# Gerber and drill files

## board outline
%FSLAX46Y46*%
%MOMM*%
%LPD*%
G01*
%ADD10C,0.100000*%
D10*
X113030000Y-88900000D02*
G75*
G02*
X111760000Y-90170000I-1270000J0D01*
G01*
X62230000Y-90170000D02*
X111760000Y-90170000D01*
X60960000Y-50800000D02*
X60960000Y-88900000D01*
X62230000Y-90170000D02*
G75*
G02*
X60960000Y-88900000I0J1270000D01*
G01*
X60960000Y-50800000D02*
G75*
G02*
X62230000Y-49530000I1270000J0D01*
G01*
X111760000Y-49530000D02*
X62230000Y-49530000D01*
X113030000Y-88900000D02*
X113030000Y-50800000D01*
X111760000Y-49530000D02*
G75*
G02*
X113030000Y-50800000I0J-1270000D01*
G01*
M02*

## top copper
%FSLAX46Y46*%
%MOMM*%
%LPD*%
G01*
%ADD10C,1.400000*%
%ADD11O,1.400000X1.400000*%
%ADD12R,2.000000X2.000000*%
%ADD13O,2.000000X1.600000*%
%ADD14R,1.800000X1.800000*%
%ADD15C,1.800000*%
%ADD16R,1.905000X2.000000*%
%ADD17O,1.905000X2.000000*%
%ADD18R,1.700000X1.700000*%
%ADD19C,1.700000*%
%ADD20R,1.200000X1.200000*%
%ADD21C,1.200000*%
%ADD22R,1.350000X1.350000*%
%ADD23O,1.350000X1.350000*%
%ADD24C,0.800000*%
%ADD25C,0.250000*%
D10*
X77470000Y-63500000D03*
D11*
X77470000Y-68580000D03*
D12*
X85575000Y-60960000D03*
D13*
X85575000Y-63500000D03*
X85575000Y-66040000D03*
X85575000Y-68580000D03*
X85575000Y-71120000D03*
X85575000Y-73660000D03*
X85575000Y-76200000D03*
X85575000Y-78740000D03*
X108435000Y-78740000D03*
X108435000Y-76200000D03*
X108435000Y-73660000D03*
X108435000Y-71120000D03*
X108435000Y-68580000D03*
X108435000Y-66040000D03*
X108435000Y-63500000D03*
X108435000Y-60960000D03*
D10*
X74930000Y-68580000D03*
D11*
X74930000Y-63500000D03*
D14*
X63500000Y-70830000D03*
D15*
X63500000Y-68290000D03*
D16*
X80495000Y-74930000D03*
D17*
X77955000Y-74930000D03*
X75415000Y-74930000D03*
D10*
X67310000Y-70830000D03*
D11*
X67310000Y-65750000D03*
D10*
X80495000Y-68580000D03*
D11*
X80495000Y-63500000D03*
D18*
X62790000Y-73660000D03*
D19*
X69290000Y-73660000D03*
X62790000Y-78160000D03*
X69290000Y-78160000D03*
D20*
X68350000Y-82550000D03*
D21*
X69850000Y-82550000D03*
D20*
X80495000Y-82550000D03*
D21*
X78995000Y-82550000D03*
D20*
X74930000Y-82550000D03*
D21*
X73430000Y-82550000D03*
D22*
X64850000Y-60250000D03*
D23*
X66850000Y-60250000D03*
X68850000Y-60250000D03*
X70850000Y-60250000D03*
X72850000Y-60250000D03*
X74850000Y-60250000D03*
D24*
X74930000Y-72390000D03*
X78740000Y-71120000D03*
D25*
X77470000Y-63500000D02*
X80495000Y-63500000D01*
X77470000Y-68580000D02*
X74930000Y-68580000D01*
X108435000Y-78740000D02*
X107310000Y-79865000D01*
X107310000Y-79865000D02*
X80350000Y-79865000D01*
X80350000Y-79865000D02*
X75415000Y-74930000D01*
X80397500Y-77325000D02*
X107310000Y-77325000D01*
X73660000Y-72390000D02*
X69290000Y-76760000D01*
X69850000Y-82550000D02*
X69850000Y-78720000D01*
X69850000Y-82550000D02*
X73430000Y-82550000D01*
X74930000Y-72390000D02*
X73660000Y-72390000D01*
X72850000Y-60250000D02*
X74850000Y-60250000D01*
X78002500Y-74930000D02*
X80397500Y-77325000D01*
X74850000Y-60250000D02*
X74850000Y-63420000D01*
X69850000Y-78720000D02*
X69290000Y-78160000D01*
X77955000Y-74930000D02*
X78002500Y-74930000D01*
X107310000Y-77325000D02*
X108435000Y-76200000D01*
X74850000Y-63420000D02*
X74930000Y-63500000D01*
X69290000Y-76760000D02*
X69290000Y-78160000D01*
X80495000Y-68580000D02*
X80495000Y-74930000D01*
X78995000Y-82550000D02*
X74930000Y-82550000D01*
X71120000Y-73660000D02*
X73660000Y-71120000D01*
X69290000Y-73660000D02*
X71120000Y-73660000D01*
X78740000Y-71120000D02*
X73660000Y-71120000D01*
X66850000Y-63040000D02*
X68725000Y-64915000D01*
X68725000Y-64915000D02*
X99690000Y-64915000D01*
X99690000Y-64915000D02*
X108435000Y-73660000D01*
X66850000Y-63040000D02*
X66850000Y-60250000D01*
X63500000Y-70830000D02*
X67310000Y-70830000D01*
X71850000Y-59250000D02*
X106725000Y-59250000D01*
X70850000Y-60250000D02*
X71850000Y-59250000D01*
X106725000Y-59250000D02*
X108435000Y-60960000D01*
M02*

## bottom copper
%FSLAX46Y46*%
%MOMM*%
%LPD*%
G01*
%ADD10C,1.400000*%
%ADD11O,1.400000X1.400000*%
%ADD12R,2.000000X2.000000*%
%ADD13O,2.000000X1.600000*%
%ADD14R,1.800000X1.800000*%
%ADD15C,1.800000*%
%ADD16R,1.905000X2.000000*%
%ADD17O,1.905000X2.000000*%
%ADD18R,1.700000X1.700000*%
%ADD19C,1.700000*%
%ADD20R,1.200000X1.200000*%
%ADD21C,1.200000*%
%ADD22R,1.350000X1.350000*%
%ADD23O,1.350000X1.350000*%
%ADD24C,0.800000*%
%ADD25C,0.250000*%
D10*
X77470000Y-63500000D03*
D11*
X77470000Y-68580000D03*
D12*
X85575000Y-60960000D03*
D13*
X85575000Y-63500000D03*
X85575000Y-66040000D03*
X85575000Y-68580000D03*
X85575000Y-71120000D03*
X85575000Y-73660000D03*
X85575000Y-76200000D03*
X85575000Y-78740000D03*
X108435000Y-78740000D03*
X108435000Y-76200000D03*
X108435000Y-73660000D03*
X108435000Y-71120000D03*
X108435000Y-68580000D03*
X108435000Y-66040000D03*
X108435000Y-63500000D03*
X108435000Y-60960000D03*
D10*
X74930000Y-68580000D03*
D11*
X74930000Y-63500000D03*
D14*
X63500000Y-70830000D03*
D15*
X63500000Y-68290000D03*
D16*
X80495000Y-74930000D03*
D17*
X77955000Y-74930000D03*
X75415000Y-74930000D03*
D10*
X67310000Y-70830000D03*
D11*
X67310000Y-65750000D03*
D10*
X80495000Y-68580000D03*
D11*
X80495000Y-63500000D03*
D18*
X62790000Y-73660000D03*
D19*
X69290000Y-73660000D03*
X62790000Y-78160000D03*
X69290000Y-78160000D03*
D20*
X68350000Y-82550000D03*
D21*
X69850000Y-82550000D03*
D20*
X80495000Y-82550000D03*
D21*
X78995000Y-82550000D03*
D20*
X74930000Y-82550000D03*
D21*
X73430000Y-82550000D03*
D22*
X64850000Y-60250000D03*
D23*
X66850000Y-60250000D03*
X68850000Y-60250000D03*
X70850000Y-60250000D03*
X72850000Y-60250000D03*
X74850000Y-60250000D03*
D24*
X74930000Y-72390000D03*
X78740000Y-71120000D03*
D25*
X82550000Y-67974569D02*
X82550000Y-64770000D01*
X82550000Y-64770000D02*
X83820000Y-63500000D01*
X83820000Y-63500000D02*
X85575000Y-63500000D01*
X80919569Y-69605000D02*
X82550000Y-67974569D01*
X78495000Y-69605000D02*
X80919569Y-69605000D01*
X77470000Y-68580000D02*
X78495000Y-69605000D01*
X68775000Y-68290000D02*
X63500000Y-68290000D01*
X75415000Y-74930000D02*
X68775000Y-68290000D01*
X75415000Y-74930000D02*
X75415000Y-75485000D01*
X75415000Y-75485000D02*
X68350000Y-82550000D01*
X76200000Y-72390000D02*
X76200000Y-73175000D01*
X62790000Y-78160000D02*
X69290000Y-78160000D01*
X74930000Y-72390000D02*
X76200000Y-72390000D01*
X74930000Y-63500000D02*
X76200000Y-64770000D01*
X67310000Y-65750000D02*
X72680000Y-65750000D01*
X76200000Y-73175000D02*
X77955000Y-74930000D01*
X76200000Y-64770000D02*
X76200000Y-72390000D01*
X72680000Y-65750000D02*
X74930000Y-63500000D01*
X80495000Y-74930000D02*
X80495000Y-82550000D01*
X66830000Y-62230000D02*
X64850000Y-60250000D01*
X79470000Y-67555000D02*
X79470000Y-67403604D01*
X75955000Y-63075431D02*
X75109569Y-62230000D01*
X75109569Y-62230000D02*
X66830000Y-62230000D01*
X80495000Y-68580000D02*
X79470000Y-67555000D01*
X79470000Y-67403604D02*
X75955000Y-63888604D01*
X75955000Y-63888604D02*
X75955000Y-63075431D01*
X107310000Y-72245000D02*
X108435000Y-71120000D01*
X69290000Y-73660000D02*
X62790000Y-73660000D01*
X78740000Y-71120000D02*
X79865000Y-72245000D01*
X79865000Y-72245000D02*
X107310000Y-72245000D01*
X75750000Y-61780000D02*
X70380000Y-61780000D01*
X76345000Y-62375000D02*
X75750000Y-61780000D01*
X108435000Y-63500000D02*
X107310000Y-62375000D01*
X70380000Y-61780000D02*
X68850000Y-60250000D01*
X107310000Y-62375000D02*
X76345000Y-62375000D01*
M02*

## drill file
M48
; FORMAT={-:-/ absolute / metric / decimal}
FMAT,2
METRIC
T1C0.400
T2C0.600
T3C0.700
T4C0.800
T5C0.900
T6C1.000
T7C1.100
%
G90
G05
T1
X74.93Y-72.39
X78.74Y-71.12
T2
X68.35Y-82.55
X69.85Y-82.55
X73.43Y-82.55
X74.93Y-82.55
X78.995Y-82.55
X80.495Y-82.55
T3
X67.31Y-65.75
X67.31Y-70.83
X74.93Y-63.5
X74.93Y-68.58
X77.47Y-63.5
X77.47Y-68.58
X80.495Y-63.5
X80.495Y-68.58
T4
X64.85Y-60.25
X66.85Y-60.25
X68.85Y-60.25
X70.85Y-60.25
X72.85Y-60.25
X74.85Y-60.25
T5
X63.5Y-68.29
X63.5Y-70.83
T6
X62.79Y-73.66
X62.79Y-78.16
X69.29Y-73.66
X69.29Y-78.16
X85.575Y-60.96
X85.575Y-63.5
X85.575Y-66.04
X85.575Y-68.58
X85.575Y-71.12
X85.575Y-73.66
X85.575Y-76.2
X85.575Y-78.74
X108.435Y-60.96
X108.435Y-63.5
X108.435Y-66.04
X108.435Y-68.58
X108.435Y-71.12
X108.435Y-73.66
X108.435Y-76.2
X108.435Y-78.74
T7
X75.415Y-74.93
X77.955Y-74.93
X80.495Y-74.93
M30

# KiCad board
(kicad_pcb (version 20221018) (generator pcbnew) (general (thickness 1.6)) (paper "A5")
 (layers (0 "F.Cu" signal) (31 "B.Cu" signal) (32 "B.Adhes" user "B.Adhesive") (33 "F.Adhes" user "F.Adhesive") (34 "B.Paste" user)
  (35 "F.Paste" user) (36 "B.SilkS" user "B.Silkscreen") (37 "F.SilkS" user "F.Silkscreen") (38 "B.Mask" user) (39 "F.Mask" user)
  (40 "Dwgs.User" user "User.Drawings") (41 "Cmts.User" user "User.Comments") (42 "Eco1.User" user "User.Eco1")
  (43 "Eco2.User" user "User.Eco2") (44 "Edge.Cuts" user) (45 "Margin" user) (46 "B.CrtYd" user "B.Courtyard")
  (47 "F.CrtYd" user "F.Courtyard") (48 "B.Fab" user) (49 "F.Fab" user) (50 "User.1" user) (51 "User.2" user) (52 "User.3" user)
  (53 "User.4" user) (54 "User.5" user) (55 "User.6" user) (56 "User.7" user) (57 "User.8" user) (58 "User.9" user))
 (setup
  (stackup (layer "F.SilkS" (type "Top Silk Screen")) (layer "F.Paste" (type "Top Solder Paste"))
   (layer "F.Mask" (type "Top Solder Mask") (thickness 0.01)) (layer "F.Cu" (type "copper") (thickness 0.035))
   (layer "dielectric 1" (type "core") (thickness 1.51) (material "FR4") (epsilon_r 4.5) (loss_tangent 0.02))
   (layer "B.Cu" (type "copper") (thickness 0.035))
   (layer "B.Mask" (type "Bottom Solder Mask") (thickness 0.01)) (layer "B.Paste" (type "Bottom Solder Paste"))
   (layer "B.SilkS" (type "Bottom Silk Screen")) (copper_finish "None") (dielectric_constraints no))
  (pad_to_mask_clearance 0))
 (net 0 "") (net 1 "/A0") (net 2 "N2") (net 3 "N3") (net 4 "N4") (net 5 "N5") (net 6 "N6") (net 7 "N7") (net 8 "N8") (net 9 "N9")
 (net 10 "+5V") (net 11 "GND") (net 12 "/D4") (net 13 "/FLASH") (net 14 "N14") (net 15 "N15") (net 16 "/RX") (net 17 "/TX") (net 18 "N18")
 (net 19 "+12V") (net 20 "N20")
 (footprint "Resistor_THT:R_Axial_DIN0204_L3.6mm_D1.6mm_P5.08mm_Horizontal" (layer "F.Cu") (at 77.47 63.5 -90)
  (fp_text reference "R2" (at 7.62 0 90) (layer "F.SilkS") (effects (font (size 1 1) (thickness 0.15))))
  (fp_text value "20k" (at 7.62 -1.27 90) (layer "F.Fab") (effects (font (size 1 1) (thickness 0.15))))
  (pad "1" thru_hole circle (at 0 0 270) (size 1.4 1.4) (drill 0.7) (layers "*.Cu" "*.Mask") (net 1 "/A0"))
  (pad "2" thru_hole oval (at 5.08 0 270) (size 1.4 1.4) (drill 0.7) (layers "*.Cu" "*.Mask") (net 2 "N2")))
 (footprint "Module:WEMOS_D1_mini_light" (layer "F.Cu") (at 85.575 60.96)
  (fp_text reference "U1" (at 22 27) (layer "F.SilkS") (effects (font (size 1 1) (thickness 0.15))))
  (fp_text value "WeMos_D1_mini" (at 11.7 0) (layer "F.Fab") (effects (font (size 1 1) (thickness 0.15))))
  (pad "1" thru_hole rect (at 0 0) (size 2 2) (drill 1) (layers "*.Cu" "*.Mask") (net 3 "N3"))
  (pad "2" thru_hole oval (at 0 2.54) (size 2 1.6) (drill 1) (layers "*.Cu" "*.Mask") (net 1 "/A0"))
  (pad "3" thru_hole oval (at 0 5.08) (size 2 1.6) (drill 1) (layers "*.Cu" "*.Mask") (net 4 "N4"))
  (pad "4" thru_hole oval (at 0 7.62) (size 2 1.6) (drill 1) (layers "*.Cu" "*.Mask") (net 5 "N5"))
  (pad "5" thru_hole oval (at 0 10.16) (size 2 1.6) (drill 1) (layers "*.Cu" "*.Mask") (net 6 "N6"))
  (pad "6" thru_hole oval (at 0 12.7) (size 2 1.6) (drill 1) (layers "*.Cu" "*.Mask") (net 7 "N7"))
  (pad "7" thru_hole oval (at 0 15.24) (size 2 1.6) (drill 1) (layers "*.Cu" "*.Mask") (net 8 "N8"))
  (pad "8" thru_hole oval (at 0 17.78) (size 2 1.6) (drill 1) (layers "*.Cu" "*.Mask") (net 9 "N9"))
  (pad "9" thru_hole oval (at 22.86 17.78) (size 2 1.6) (drill 1) (layers "*.Cu" "*.Mask") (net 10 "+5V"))
  (pad "10" thru_hole oval (at 22.86 15.24) (size 2 1.6) (drill 1) (layers "*.Cu" "*.Mask") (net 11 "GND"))
  (pad "11" thru_hole oval (at 22.86 12.7) (size 2 1.6) (drill 1) (layers "*.Cu" "*.Mask") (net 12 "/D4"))
  (pad "12" thru_hole oval (at 22.86 10.16) (size 2 1.6) (drill 1) (layers "*.Cu" "*.Mask") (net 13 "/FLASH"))
  (pad "13" thru_hole oval (at 22.86 7.62) (size 2 1.6) (drill 1) (layers "*.Cu" "*.Mask") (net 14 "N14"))
  (pad "14" thru_hole oval (at 22.86 5.08) (size 2 1.6) (drill 1) (layers "*.Cu" "*.Mask") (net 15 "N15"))
  (pad "15" thru_hole oval (at 22.86 2.54) (size 2 1.6) (drill 1) (layers "*.Cu" "*.Mask") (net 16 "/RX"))
  (pad "16" thru_hole oval (at 22.86 0) (size 2 1.6) (drill 1) (layers "*.Cu" "*.Mask") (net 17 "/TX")))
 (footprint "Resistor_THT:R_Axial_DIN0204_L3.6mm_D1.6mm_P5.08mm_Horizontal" (layer "F.Cu") (at 74.93 68.58 90)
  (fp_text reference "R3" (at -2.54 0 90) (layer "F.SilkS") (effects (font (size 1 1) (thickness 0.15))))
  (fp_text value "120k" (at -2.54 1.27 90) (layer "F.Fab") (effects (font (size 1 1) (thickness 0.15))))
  (pad "1" thru_hole circle (at 0 0 90) (size 1.4 1.4) (drill 0.7) (layers "*.Cu" "*.Mask") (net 2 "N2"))
  (pad "2" thru_hole oval (at 5.08 0 90) (size 1.4 1.4) (drill 0.7) (layers "*.Cu" "*.Mask") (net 11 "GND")))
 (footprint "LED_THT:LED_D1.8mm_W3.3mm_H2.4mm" (layer "F.Cu") (at 63.5 70.83 90)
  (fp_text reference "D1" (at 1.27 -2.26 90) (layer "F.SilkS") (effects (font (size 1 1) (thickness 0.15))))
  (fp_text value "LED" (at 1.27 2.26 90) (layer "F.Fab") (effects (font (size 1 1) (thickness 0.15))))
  (pad "1" thru_hole rect (at 0 0 90) (size 1.8 1.8) (drill 0.9) (layers "*.Cu" "*.Mask") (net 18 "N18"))
  (pad "2" thru_hole circle (at 2.54 0 90) (size 1.8 1.8) (drill 0.9) (layers "*.Cu" "*.Mask") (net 10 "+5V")))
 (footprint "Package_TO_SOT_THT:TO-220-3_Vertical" (layer "F.Cu") (at 80.495 74.93 180)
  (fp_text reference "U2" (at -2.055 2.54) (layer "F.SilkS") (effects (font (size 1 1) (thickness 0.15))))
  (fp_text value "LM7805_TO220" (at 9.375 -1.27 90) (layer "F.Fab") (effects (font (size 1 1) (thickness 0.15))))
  (pad "1" thru_hole rect (at 0 0 180) (size 1.905 2) (drill 1.1) (layers "*.Cu" "*.Mask") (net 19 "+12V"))
  (pad "2" thru_hole oval (at 2.54 0 180) (size 1.905 2) (drill 1.1) (layers "*.Cu" "*.Mask") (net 11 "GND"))
  (pad "3" thru_hole oval (at 5.08 0 180) (size 1.905 2) (drill 1.1) (layers "*.Cu" "*.Mask") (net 10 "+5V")))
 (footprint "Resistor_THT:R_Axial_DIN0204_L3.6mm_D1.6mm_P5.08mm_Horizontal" (layer "F.Cu") (at 67.31 70.83 90)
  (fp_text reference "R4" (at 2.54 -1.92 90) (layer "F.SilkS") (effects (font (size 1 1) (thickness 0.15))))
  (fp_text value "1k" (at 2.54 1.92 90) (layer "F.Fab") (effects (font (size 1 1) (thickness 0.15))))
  (pad "1" thru_hole circle (at 0 0 90) (size 1.4 1.4) (drill 0.7) (layers "*.Cu" "*.Mask") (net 18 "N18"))
  (pad "2" thru_hole oval (at 5.08 0 90) (size 1.4 1.4) (drill 0.7) (layers "*.Cu" "*.Mask") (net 11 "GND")))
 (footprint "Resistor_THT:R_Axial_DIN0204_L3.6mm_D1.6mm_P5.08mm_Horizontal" (layer "F.Cu") (at 80.495 68.58 90)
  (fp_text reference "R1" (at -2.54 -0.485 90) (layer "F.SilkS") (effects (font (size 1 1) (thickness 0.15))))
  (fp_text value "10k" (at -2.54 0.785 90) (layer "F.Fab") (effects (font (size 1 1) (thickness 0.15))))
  (pad "1" thru_hole circle (at 0 0 90) (size 1.4 1.4) (drill 0.7) (layers "*.Cu" "*.Mask") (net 19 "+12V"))
  (pad "2" thru_hole oval (at 5.08 0 90) (size 1.4 1.4) (drill 0.7) (layers "*.Cu" "*.Mask") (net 1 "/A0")))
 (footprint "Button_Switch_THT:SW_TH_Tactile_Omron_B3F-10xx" (layer "F.Cu") (at 62.79 73.66)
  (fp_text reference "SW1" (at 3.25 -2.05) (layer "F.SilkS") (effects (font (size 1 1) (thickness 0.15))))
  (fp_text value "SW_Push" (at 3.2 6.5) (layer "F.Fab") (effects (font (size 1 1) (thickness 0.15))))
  (pad "1" thru_hole rect (at 0 0) (size 1.7 1.7) (drill 1) (layers "*.Cu" "*.Mask") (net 13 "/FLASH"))
  (pad "1" thru_hole circle (at 6.5 0) (size 1.7 1.7) (drill 1) (layers "*.Cu" "*.Mask") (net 13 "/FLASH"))
  (pad "2" thru_hole circle (at 0 4.5) (size 1.7 1.7) (drill 1) (layers "*.Cu" "*.Mask") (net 11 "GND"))
  (pad "2" thru_hole circle (at 6.5 4.5) (size 1.7 1.7) (drill 1) (layers "*.Cu" "*.Mask") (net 11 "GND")))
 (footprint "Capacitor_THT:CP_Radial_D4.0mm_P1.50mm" (layer "F.Cu") (at 68.35 82.55)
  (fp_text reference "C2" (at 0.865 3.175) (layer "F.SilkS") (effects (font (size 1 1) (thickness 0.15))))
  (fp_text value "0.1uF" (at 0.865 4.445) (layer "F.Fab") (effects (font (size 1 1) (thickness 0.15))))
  (pad "1" thru_hole rect (at 0 0) (size 1.2 1.2) (drill 0.6) (layers "*.Cu" "*.Mask") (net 10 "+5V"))
  (pad "2" thru_hole circle (at 1.5 0) (size 1.2 1.2) (drill 0.6) (layers "*.Cu" "*.Mask") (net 11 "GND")))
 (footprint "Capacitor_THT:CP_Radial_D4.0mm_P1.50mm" (layer "F.Cu") (at 80.495 82.55 180)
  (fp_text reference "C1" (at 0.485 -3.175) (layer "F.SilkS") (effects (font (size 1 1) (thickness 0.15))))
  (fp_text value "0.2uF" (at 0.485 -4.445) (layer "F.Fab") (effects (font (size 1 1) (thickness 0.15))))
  (pad "1" thru_hole rect (at 0 0 180) (size 1.2 1.2) (drill 0.6) (layers "*.Cu" "*.Mask") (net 19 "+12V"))
  (pad "2" thru_hole circle (at 1.5 0 180) (size 1.2 1.2) (drill 0.6) (layers "*.Cu" "*.Mask") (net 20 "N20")))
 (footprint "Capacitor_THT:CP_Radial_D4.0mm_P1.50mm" (layer "F.Cu") (at 74.93 82.55 180)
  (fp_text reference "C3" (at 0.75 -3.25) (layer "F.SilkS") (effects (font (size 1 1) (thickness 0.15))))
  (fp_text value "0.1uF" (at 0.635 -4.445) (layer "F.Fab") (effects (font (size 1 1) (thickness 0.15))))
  (pad "1" thru_hole rect (at 0 0 180) (size 1.2 1.2) (drill 0.6) (layers "*.Cu" "*.Mask") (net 20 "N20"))
  (pad "2" thru_hole circle (at 1.5 0 180) (size 1.2 1.2) (drill 0.6) (layers "*.Cu" "*.Mask") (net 11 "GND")))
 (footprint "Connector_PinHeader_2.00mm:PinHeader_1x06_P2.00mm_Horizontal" (layer "F.Cu") (at 64.85 60.25 90)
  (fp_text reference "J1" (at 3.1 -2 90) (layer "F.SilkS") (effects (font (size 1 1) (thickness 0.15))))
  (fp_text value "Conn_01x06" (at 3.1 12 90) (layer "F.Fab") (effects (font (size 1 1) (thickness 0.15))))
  (pad "1" thru_hole rect (at 0 0 90) (size 1.35 1.35) (drill 0.8) (layers "*.Cu" "*.Mask") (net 19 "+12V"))
  (pad "2" thru_hole oval (at 0 2 90) (size 1.35 1.35) (drill 0.8) (layers "*.Cu" "*.Mask") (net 12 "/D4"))
  (pad "3" thru_hole oval (at 0 4 90) (size 1.35 1.35) (drill 0.8) (layers "*.Cu" "*.Mask") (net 16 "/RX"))
  (pad "4" thru_hole oval (at 0 6 90) (size 1.35 1.35) (drill 0.8) (layers "*.Cu" "*.Mask") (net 17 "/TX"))
  (pad "5" thru_hole oval (at 0 8 90) (size 1.35 1.35) (drill 0.8) (layers "*.Cu" "*.Mask") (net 11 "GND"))
  (pad "6" thru_hole oval (at 0 10 90) (size 1.35 1.35) (drill 0.8) (layers "*.Cu" "*.Mask") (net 11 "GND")))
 (gr_arc locked (start 113.03 88.9) (mid 112.658026 89.798026) (end 111.76 90.17) (stroke (width 0.1) (type default)) (layer "Edge.Cuts"))
 (gr_line locked (start 62.23 90.17) (end 111.76 90.17) (stroke (width 0.1) (type default)) (layer "Edge.Cuts"))
 (gr_line locked (start 60.96 50.8) (end 60.96 88.9) (stroke (width 0.1) (type default)) (layer "Edge.Cuts"))
 (gr_arc locked (start 62.23 90.17) (mid 61.331974 89.798026) (end 60.96 88.9) (stroke (width 0.1) (type default)) (layer "Edge.Cuts"))
 (gr_arc locked (start 60.96 50.8) (mid 61.331974 49.901974) (end 62.23 49.53) (stroke (width 0.1) (type default)) (layer "Edge.Cuts"))
 (gr_line locked (start 111.76 49.53) (end 62.23 49.53) (stroke (width 0.1) (type default)) (layer "Edge.Cuts"))
 (gr_line locked (start 113.03 88.9) (end 113.03 50.8) (stroke (width 0.1) (type default)) (layer "Edge.Cuts"))
 (gr_arc locked (start 111.76 49.53) (mid 112.658026 49.901974) (end 113.03 50.8) (stroke (width 0.1) (type default)) (layer "Edge.Cuts"))
 (segment (start 77.47 63.5) (end 80.495 63.5) (width 0.25) (layer "F.Cu") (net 1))
 (segment (start 77.47 68.58) (end 74.93 68.58) (width 0.25) (layer "F.Cu") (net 1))
 (segment (start 82.55 67.974569) (end 82.55 64.77) (width 0.25) (layer "B.Cu") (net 1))
 (segment (start 82.55 64.77) (end 83.82 63.5) (width 0.25) (layer "B.Cu") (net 1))
 (segment (start 83.82 63.5) (end 85.575 63.5) (width 0.25) (layer "B.Cu") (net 1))
 (segment (start 80.919569 69.605) (end 82.55 67.974569) (width 0.25) (layer "B.Cu") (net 1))
 (segment (start 78.495 69.605) (end 80.919569 69.605) (width 0.25) (layer "B.Cu") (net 1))
 (segment (start 77.47 68.58) (end 78.495 69.605) (width 0.25) (layer "B.Cu") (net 1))
 (segment (start 108.435 78.74) (end 107.31 79.865) (width 0.25) (layer "F.Cu") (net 10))
 (segment (start 107.31 79.865) (end 80.35 79.865) (width 0.25) (layer "F.Cu") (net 10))
 (segment (start 80.35 79.865) (end 75.415 74.93) (width 0.25) (layer "F.Cu") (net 10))
 (segment (start 68.775 68.29) (end 63.5 68.29) (width 0.25) (layer "B.Cu") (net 10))
 (segment (start 75.415 74.93) (end 68.775 68.29) (width 0.25) (layer "B.Cu") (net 10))
 (segment (start 75.415 74.93) (end 75.415 75.485) (width 0.25) (layer "B.Cu") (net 10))
 (segment (start 75.415 75.485) (end 68.35 82.55) (width 0.25) (layer "B.Cu") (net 10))
 (segment (start 80.3975 77.325) (end 107.31 77.325) (width 0.25) (layer "F.Cu") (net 11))
 (segment (start 73.66 72.39) (end 69.29 76.76) (width 0.25) (layer "F.Cu") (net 11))
 (segment (start 69.85 82.55) (end 69.85 78.72) (width 0.25) (layer "F.Cu") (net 11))
 (segment (start 69.85 82.55) (end 73.43 82.55) (width 0.25) (layer "F.Cu") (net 11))
 (segment (start 74.93 72.39) (end 73.66 72.39) (width 0.25) (layer "F.Cu") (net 11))
 (segment (start 72.85 60.25) (end 74.85 60.25) (width 0.25) (layer "F.Cu") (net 11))
 (segment (start 78.0025 74.93) (end 80.3975 77.325) (width 0.25) (layer "F.Cu") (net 11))
 (segment (start 74.85 60.25) (end 74.85 63.42) (width 0.25) (layer "F.Cu") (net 11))
 (segment (start 69.85 78.72) (end 69.29 78.16) (width 0.25) (layer "F.Cu") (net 11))
 (segment (start 77.955 74.93) (end 78.0025 74.93) (width 0.25) (layer "F.Cu") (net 11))
 (segment (start 107.31 77.325) (end 108.435 76.2) (width 0.25) (layer "F.Cu") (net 11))
 (segment (start 74.85 63.42) (end 74.93 63.5) (width 0.25) (layer "F.Cu") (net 11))
 (segment (start 69.29 76.76) (end 69.29 78.16) (width 0.25) (layer "F.Cu") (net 11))
 (via (at 74.93 72.39) (size 0.8) (drill 0.4) (layers "F.Cu" "B.Cu") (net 11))
 (segment (start 76.2 72.39) (end 76.2 73.175) (width 0.25) (layer "B.Cu") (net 11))
 (segment (start 62.79 78.16) (end 69.29 78.16) (width 0.25) (layer "B.Cu") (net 11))
 (segment (start 74.93 72.39) (end 76.2 72.39) (width 0.25) (layer "B.Cu") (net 11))
 (segment (start 74.93 63.5) (end 76.2 64.77) (width 0.25) (layer "B.Cu") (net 11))
 (segment (start 67.31 65.75) (end 72.68 65.75) (width 0.25) (layer "B.Cu") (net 11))
 (segment (start 76.2 73.175) (end 77.955 74.93) (width 0.25) (layer "B.Cu") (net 11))
 (segment (start 76.2 64.77) (end 76.2 72.39) (width 0.25) (layer "B.Cu") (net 11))
 (segment (start 72.68 65.75) (end 74.93 63.5) (width 0.25) (layer "B.Cu") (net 11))
 (segment (start 80.495 68.58) (end 80.495 74.93) (width 0.25) (layer "F.Cu") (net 19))
 (segment (start 80.495 74.93) (end 80.495 82.55) (width 0.25) (layer "B.Cu") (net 19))
 (segment (start 66.83 62.23) (end 64.85 60.25) (width 0.25) (layer "B.Cu") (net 19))
 (segment (start 79.47 67.555) (end 79.47 67.403604) (width 0.25) (layer "B.Cu") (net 19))
 (segment (start 75.955 63.075431) (end 75.109569 62.23) (width 0.25) (layer "B.Cu") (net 19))
 (segment (start 75.109569 62.23) (end 66.83 62.23) (width 0.25) (layer "B.Cu") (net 19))
 (segment (start 80.495 68.58) (end 79.47 67.555) (width 0.25) (layer "B.Cu") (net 19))
 (segment (start 79.47 67.403604) (end 75.955 63.888604) (width 0.25) (layer "B.Cu") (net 19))
 (segment (start 75.955 63.888604) (end 75.955 63.075431) (width 0.25) (layer "B.Cu") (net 19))
 (segment (start 78.995 82.55) (end 74.93 82.55) (width 0.25) (layer "F.Cu") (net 20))
 (segment (start 71.12 73.66) (end 73.66 71.12) (width 0.25) (layer "F.Cu") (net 13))
 (segment (start 69.29 73.66) (end 71.12 73.66) (width 0.25) (layer "F.Cu") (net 13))
 (segment (start 78.74 71.12) (end 73.66 71.12) (width 0.25) (layer "F.Cu") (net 13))
 (via (at 78.74 71.12) (size 0.8) (drill 0.4) (layers "F.Cu" "B.Cu") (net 13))
 (segment (start 107.31 72.245) (end 108.435 71.12) (width 0.25) (layer "B.Cu") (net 13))
 (segment (start 69.29 73.66) (end 62.79 73.66) (width 0.25) (layer "B.Cu") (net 13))
 (segment (start 78.74 71.12) (end 79.865 72.245) (width 0.25) (layer "B.Cu") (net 13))
 (segment (start 79.865 72.245) (end 107.31 72.245) (width 0.25) (layer "B.Cu") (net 13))
 (segment (start 66.85 63.04) (end 68.725 64.915) (width 0.25) (layer "F.Cu") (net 12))
 (segment (start 68.725 64.915) (end 99.69 64.915) (width 0.25) (layer "F.Cu") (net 12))
 (segment (start 99.69 64.915) (end 108.435 73.66) (width 0.25) (layer "F.Cu") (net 12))
 (segment (start 66.85 63.04) (end 66.85 60.25) (width 0.25) (layer "F.Cu") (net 12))
 (segment (start 63.5 70.83) (end 67.31 70.83) (width 0.25) (layer "F.Cu") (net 18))
 (segment (start 75.75 61.78) (end 70.38 61.78) (width 0.25) (layer "B.Cu") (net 16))
 (segment (start 76.345 62.375) (end 75.75 61.78) (width 0.25) (layer "B.Cu") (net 16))
 (segment (start 108.435 63.5) (end 107.31 62.375) (width 0.25) (layer "B.Cu") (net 16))
 (segment (start 70.38 61.78) (end 68.85 60.25) (width 0.25) (layer "B.Cu") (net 16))
 (segment (start 107.31 62.375) (end 76.345 62.375) (width 0.25) (layer "B.Cu") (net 16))
 (segment (start 71.85 59.25) (end 106.725 59.25) (width 0.25) (layer "F.Cu") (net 17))
 (segment (start 70.85 60.25) (end 71.85 59.25) (width 0.25) (layer "F.Cu") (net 17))
 (segment (start 106.725 59.25) (end 108.435 60.96) (width 0.25) (layer "F.Cu") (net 17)))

